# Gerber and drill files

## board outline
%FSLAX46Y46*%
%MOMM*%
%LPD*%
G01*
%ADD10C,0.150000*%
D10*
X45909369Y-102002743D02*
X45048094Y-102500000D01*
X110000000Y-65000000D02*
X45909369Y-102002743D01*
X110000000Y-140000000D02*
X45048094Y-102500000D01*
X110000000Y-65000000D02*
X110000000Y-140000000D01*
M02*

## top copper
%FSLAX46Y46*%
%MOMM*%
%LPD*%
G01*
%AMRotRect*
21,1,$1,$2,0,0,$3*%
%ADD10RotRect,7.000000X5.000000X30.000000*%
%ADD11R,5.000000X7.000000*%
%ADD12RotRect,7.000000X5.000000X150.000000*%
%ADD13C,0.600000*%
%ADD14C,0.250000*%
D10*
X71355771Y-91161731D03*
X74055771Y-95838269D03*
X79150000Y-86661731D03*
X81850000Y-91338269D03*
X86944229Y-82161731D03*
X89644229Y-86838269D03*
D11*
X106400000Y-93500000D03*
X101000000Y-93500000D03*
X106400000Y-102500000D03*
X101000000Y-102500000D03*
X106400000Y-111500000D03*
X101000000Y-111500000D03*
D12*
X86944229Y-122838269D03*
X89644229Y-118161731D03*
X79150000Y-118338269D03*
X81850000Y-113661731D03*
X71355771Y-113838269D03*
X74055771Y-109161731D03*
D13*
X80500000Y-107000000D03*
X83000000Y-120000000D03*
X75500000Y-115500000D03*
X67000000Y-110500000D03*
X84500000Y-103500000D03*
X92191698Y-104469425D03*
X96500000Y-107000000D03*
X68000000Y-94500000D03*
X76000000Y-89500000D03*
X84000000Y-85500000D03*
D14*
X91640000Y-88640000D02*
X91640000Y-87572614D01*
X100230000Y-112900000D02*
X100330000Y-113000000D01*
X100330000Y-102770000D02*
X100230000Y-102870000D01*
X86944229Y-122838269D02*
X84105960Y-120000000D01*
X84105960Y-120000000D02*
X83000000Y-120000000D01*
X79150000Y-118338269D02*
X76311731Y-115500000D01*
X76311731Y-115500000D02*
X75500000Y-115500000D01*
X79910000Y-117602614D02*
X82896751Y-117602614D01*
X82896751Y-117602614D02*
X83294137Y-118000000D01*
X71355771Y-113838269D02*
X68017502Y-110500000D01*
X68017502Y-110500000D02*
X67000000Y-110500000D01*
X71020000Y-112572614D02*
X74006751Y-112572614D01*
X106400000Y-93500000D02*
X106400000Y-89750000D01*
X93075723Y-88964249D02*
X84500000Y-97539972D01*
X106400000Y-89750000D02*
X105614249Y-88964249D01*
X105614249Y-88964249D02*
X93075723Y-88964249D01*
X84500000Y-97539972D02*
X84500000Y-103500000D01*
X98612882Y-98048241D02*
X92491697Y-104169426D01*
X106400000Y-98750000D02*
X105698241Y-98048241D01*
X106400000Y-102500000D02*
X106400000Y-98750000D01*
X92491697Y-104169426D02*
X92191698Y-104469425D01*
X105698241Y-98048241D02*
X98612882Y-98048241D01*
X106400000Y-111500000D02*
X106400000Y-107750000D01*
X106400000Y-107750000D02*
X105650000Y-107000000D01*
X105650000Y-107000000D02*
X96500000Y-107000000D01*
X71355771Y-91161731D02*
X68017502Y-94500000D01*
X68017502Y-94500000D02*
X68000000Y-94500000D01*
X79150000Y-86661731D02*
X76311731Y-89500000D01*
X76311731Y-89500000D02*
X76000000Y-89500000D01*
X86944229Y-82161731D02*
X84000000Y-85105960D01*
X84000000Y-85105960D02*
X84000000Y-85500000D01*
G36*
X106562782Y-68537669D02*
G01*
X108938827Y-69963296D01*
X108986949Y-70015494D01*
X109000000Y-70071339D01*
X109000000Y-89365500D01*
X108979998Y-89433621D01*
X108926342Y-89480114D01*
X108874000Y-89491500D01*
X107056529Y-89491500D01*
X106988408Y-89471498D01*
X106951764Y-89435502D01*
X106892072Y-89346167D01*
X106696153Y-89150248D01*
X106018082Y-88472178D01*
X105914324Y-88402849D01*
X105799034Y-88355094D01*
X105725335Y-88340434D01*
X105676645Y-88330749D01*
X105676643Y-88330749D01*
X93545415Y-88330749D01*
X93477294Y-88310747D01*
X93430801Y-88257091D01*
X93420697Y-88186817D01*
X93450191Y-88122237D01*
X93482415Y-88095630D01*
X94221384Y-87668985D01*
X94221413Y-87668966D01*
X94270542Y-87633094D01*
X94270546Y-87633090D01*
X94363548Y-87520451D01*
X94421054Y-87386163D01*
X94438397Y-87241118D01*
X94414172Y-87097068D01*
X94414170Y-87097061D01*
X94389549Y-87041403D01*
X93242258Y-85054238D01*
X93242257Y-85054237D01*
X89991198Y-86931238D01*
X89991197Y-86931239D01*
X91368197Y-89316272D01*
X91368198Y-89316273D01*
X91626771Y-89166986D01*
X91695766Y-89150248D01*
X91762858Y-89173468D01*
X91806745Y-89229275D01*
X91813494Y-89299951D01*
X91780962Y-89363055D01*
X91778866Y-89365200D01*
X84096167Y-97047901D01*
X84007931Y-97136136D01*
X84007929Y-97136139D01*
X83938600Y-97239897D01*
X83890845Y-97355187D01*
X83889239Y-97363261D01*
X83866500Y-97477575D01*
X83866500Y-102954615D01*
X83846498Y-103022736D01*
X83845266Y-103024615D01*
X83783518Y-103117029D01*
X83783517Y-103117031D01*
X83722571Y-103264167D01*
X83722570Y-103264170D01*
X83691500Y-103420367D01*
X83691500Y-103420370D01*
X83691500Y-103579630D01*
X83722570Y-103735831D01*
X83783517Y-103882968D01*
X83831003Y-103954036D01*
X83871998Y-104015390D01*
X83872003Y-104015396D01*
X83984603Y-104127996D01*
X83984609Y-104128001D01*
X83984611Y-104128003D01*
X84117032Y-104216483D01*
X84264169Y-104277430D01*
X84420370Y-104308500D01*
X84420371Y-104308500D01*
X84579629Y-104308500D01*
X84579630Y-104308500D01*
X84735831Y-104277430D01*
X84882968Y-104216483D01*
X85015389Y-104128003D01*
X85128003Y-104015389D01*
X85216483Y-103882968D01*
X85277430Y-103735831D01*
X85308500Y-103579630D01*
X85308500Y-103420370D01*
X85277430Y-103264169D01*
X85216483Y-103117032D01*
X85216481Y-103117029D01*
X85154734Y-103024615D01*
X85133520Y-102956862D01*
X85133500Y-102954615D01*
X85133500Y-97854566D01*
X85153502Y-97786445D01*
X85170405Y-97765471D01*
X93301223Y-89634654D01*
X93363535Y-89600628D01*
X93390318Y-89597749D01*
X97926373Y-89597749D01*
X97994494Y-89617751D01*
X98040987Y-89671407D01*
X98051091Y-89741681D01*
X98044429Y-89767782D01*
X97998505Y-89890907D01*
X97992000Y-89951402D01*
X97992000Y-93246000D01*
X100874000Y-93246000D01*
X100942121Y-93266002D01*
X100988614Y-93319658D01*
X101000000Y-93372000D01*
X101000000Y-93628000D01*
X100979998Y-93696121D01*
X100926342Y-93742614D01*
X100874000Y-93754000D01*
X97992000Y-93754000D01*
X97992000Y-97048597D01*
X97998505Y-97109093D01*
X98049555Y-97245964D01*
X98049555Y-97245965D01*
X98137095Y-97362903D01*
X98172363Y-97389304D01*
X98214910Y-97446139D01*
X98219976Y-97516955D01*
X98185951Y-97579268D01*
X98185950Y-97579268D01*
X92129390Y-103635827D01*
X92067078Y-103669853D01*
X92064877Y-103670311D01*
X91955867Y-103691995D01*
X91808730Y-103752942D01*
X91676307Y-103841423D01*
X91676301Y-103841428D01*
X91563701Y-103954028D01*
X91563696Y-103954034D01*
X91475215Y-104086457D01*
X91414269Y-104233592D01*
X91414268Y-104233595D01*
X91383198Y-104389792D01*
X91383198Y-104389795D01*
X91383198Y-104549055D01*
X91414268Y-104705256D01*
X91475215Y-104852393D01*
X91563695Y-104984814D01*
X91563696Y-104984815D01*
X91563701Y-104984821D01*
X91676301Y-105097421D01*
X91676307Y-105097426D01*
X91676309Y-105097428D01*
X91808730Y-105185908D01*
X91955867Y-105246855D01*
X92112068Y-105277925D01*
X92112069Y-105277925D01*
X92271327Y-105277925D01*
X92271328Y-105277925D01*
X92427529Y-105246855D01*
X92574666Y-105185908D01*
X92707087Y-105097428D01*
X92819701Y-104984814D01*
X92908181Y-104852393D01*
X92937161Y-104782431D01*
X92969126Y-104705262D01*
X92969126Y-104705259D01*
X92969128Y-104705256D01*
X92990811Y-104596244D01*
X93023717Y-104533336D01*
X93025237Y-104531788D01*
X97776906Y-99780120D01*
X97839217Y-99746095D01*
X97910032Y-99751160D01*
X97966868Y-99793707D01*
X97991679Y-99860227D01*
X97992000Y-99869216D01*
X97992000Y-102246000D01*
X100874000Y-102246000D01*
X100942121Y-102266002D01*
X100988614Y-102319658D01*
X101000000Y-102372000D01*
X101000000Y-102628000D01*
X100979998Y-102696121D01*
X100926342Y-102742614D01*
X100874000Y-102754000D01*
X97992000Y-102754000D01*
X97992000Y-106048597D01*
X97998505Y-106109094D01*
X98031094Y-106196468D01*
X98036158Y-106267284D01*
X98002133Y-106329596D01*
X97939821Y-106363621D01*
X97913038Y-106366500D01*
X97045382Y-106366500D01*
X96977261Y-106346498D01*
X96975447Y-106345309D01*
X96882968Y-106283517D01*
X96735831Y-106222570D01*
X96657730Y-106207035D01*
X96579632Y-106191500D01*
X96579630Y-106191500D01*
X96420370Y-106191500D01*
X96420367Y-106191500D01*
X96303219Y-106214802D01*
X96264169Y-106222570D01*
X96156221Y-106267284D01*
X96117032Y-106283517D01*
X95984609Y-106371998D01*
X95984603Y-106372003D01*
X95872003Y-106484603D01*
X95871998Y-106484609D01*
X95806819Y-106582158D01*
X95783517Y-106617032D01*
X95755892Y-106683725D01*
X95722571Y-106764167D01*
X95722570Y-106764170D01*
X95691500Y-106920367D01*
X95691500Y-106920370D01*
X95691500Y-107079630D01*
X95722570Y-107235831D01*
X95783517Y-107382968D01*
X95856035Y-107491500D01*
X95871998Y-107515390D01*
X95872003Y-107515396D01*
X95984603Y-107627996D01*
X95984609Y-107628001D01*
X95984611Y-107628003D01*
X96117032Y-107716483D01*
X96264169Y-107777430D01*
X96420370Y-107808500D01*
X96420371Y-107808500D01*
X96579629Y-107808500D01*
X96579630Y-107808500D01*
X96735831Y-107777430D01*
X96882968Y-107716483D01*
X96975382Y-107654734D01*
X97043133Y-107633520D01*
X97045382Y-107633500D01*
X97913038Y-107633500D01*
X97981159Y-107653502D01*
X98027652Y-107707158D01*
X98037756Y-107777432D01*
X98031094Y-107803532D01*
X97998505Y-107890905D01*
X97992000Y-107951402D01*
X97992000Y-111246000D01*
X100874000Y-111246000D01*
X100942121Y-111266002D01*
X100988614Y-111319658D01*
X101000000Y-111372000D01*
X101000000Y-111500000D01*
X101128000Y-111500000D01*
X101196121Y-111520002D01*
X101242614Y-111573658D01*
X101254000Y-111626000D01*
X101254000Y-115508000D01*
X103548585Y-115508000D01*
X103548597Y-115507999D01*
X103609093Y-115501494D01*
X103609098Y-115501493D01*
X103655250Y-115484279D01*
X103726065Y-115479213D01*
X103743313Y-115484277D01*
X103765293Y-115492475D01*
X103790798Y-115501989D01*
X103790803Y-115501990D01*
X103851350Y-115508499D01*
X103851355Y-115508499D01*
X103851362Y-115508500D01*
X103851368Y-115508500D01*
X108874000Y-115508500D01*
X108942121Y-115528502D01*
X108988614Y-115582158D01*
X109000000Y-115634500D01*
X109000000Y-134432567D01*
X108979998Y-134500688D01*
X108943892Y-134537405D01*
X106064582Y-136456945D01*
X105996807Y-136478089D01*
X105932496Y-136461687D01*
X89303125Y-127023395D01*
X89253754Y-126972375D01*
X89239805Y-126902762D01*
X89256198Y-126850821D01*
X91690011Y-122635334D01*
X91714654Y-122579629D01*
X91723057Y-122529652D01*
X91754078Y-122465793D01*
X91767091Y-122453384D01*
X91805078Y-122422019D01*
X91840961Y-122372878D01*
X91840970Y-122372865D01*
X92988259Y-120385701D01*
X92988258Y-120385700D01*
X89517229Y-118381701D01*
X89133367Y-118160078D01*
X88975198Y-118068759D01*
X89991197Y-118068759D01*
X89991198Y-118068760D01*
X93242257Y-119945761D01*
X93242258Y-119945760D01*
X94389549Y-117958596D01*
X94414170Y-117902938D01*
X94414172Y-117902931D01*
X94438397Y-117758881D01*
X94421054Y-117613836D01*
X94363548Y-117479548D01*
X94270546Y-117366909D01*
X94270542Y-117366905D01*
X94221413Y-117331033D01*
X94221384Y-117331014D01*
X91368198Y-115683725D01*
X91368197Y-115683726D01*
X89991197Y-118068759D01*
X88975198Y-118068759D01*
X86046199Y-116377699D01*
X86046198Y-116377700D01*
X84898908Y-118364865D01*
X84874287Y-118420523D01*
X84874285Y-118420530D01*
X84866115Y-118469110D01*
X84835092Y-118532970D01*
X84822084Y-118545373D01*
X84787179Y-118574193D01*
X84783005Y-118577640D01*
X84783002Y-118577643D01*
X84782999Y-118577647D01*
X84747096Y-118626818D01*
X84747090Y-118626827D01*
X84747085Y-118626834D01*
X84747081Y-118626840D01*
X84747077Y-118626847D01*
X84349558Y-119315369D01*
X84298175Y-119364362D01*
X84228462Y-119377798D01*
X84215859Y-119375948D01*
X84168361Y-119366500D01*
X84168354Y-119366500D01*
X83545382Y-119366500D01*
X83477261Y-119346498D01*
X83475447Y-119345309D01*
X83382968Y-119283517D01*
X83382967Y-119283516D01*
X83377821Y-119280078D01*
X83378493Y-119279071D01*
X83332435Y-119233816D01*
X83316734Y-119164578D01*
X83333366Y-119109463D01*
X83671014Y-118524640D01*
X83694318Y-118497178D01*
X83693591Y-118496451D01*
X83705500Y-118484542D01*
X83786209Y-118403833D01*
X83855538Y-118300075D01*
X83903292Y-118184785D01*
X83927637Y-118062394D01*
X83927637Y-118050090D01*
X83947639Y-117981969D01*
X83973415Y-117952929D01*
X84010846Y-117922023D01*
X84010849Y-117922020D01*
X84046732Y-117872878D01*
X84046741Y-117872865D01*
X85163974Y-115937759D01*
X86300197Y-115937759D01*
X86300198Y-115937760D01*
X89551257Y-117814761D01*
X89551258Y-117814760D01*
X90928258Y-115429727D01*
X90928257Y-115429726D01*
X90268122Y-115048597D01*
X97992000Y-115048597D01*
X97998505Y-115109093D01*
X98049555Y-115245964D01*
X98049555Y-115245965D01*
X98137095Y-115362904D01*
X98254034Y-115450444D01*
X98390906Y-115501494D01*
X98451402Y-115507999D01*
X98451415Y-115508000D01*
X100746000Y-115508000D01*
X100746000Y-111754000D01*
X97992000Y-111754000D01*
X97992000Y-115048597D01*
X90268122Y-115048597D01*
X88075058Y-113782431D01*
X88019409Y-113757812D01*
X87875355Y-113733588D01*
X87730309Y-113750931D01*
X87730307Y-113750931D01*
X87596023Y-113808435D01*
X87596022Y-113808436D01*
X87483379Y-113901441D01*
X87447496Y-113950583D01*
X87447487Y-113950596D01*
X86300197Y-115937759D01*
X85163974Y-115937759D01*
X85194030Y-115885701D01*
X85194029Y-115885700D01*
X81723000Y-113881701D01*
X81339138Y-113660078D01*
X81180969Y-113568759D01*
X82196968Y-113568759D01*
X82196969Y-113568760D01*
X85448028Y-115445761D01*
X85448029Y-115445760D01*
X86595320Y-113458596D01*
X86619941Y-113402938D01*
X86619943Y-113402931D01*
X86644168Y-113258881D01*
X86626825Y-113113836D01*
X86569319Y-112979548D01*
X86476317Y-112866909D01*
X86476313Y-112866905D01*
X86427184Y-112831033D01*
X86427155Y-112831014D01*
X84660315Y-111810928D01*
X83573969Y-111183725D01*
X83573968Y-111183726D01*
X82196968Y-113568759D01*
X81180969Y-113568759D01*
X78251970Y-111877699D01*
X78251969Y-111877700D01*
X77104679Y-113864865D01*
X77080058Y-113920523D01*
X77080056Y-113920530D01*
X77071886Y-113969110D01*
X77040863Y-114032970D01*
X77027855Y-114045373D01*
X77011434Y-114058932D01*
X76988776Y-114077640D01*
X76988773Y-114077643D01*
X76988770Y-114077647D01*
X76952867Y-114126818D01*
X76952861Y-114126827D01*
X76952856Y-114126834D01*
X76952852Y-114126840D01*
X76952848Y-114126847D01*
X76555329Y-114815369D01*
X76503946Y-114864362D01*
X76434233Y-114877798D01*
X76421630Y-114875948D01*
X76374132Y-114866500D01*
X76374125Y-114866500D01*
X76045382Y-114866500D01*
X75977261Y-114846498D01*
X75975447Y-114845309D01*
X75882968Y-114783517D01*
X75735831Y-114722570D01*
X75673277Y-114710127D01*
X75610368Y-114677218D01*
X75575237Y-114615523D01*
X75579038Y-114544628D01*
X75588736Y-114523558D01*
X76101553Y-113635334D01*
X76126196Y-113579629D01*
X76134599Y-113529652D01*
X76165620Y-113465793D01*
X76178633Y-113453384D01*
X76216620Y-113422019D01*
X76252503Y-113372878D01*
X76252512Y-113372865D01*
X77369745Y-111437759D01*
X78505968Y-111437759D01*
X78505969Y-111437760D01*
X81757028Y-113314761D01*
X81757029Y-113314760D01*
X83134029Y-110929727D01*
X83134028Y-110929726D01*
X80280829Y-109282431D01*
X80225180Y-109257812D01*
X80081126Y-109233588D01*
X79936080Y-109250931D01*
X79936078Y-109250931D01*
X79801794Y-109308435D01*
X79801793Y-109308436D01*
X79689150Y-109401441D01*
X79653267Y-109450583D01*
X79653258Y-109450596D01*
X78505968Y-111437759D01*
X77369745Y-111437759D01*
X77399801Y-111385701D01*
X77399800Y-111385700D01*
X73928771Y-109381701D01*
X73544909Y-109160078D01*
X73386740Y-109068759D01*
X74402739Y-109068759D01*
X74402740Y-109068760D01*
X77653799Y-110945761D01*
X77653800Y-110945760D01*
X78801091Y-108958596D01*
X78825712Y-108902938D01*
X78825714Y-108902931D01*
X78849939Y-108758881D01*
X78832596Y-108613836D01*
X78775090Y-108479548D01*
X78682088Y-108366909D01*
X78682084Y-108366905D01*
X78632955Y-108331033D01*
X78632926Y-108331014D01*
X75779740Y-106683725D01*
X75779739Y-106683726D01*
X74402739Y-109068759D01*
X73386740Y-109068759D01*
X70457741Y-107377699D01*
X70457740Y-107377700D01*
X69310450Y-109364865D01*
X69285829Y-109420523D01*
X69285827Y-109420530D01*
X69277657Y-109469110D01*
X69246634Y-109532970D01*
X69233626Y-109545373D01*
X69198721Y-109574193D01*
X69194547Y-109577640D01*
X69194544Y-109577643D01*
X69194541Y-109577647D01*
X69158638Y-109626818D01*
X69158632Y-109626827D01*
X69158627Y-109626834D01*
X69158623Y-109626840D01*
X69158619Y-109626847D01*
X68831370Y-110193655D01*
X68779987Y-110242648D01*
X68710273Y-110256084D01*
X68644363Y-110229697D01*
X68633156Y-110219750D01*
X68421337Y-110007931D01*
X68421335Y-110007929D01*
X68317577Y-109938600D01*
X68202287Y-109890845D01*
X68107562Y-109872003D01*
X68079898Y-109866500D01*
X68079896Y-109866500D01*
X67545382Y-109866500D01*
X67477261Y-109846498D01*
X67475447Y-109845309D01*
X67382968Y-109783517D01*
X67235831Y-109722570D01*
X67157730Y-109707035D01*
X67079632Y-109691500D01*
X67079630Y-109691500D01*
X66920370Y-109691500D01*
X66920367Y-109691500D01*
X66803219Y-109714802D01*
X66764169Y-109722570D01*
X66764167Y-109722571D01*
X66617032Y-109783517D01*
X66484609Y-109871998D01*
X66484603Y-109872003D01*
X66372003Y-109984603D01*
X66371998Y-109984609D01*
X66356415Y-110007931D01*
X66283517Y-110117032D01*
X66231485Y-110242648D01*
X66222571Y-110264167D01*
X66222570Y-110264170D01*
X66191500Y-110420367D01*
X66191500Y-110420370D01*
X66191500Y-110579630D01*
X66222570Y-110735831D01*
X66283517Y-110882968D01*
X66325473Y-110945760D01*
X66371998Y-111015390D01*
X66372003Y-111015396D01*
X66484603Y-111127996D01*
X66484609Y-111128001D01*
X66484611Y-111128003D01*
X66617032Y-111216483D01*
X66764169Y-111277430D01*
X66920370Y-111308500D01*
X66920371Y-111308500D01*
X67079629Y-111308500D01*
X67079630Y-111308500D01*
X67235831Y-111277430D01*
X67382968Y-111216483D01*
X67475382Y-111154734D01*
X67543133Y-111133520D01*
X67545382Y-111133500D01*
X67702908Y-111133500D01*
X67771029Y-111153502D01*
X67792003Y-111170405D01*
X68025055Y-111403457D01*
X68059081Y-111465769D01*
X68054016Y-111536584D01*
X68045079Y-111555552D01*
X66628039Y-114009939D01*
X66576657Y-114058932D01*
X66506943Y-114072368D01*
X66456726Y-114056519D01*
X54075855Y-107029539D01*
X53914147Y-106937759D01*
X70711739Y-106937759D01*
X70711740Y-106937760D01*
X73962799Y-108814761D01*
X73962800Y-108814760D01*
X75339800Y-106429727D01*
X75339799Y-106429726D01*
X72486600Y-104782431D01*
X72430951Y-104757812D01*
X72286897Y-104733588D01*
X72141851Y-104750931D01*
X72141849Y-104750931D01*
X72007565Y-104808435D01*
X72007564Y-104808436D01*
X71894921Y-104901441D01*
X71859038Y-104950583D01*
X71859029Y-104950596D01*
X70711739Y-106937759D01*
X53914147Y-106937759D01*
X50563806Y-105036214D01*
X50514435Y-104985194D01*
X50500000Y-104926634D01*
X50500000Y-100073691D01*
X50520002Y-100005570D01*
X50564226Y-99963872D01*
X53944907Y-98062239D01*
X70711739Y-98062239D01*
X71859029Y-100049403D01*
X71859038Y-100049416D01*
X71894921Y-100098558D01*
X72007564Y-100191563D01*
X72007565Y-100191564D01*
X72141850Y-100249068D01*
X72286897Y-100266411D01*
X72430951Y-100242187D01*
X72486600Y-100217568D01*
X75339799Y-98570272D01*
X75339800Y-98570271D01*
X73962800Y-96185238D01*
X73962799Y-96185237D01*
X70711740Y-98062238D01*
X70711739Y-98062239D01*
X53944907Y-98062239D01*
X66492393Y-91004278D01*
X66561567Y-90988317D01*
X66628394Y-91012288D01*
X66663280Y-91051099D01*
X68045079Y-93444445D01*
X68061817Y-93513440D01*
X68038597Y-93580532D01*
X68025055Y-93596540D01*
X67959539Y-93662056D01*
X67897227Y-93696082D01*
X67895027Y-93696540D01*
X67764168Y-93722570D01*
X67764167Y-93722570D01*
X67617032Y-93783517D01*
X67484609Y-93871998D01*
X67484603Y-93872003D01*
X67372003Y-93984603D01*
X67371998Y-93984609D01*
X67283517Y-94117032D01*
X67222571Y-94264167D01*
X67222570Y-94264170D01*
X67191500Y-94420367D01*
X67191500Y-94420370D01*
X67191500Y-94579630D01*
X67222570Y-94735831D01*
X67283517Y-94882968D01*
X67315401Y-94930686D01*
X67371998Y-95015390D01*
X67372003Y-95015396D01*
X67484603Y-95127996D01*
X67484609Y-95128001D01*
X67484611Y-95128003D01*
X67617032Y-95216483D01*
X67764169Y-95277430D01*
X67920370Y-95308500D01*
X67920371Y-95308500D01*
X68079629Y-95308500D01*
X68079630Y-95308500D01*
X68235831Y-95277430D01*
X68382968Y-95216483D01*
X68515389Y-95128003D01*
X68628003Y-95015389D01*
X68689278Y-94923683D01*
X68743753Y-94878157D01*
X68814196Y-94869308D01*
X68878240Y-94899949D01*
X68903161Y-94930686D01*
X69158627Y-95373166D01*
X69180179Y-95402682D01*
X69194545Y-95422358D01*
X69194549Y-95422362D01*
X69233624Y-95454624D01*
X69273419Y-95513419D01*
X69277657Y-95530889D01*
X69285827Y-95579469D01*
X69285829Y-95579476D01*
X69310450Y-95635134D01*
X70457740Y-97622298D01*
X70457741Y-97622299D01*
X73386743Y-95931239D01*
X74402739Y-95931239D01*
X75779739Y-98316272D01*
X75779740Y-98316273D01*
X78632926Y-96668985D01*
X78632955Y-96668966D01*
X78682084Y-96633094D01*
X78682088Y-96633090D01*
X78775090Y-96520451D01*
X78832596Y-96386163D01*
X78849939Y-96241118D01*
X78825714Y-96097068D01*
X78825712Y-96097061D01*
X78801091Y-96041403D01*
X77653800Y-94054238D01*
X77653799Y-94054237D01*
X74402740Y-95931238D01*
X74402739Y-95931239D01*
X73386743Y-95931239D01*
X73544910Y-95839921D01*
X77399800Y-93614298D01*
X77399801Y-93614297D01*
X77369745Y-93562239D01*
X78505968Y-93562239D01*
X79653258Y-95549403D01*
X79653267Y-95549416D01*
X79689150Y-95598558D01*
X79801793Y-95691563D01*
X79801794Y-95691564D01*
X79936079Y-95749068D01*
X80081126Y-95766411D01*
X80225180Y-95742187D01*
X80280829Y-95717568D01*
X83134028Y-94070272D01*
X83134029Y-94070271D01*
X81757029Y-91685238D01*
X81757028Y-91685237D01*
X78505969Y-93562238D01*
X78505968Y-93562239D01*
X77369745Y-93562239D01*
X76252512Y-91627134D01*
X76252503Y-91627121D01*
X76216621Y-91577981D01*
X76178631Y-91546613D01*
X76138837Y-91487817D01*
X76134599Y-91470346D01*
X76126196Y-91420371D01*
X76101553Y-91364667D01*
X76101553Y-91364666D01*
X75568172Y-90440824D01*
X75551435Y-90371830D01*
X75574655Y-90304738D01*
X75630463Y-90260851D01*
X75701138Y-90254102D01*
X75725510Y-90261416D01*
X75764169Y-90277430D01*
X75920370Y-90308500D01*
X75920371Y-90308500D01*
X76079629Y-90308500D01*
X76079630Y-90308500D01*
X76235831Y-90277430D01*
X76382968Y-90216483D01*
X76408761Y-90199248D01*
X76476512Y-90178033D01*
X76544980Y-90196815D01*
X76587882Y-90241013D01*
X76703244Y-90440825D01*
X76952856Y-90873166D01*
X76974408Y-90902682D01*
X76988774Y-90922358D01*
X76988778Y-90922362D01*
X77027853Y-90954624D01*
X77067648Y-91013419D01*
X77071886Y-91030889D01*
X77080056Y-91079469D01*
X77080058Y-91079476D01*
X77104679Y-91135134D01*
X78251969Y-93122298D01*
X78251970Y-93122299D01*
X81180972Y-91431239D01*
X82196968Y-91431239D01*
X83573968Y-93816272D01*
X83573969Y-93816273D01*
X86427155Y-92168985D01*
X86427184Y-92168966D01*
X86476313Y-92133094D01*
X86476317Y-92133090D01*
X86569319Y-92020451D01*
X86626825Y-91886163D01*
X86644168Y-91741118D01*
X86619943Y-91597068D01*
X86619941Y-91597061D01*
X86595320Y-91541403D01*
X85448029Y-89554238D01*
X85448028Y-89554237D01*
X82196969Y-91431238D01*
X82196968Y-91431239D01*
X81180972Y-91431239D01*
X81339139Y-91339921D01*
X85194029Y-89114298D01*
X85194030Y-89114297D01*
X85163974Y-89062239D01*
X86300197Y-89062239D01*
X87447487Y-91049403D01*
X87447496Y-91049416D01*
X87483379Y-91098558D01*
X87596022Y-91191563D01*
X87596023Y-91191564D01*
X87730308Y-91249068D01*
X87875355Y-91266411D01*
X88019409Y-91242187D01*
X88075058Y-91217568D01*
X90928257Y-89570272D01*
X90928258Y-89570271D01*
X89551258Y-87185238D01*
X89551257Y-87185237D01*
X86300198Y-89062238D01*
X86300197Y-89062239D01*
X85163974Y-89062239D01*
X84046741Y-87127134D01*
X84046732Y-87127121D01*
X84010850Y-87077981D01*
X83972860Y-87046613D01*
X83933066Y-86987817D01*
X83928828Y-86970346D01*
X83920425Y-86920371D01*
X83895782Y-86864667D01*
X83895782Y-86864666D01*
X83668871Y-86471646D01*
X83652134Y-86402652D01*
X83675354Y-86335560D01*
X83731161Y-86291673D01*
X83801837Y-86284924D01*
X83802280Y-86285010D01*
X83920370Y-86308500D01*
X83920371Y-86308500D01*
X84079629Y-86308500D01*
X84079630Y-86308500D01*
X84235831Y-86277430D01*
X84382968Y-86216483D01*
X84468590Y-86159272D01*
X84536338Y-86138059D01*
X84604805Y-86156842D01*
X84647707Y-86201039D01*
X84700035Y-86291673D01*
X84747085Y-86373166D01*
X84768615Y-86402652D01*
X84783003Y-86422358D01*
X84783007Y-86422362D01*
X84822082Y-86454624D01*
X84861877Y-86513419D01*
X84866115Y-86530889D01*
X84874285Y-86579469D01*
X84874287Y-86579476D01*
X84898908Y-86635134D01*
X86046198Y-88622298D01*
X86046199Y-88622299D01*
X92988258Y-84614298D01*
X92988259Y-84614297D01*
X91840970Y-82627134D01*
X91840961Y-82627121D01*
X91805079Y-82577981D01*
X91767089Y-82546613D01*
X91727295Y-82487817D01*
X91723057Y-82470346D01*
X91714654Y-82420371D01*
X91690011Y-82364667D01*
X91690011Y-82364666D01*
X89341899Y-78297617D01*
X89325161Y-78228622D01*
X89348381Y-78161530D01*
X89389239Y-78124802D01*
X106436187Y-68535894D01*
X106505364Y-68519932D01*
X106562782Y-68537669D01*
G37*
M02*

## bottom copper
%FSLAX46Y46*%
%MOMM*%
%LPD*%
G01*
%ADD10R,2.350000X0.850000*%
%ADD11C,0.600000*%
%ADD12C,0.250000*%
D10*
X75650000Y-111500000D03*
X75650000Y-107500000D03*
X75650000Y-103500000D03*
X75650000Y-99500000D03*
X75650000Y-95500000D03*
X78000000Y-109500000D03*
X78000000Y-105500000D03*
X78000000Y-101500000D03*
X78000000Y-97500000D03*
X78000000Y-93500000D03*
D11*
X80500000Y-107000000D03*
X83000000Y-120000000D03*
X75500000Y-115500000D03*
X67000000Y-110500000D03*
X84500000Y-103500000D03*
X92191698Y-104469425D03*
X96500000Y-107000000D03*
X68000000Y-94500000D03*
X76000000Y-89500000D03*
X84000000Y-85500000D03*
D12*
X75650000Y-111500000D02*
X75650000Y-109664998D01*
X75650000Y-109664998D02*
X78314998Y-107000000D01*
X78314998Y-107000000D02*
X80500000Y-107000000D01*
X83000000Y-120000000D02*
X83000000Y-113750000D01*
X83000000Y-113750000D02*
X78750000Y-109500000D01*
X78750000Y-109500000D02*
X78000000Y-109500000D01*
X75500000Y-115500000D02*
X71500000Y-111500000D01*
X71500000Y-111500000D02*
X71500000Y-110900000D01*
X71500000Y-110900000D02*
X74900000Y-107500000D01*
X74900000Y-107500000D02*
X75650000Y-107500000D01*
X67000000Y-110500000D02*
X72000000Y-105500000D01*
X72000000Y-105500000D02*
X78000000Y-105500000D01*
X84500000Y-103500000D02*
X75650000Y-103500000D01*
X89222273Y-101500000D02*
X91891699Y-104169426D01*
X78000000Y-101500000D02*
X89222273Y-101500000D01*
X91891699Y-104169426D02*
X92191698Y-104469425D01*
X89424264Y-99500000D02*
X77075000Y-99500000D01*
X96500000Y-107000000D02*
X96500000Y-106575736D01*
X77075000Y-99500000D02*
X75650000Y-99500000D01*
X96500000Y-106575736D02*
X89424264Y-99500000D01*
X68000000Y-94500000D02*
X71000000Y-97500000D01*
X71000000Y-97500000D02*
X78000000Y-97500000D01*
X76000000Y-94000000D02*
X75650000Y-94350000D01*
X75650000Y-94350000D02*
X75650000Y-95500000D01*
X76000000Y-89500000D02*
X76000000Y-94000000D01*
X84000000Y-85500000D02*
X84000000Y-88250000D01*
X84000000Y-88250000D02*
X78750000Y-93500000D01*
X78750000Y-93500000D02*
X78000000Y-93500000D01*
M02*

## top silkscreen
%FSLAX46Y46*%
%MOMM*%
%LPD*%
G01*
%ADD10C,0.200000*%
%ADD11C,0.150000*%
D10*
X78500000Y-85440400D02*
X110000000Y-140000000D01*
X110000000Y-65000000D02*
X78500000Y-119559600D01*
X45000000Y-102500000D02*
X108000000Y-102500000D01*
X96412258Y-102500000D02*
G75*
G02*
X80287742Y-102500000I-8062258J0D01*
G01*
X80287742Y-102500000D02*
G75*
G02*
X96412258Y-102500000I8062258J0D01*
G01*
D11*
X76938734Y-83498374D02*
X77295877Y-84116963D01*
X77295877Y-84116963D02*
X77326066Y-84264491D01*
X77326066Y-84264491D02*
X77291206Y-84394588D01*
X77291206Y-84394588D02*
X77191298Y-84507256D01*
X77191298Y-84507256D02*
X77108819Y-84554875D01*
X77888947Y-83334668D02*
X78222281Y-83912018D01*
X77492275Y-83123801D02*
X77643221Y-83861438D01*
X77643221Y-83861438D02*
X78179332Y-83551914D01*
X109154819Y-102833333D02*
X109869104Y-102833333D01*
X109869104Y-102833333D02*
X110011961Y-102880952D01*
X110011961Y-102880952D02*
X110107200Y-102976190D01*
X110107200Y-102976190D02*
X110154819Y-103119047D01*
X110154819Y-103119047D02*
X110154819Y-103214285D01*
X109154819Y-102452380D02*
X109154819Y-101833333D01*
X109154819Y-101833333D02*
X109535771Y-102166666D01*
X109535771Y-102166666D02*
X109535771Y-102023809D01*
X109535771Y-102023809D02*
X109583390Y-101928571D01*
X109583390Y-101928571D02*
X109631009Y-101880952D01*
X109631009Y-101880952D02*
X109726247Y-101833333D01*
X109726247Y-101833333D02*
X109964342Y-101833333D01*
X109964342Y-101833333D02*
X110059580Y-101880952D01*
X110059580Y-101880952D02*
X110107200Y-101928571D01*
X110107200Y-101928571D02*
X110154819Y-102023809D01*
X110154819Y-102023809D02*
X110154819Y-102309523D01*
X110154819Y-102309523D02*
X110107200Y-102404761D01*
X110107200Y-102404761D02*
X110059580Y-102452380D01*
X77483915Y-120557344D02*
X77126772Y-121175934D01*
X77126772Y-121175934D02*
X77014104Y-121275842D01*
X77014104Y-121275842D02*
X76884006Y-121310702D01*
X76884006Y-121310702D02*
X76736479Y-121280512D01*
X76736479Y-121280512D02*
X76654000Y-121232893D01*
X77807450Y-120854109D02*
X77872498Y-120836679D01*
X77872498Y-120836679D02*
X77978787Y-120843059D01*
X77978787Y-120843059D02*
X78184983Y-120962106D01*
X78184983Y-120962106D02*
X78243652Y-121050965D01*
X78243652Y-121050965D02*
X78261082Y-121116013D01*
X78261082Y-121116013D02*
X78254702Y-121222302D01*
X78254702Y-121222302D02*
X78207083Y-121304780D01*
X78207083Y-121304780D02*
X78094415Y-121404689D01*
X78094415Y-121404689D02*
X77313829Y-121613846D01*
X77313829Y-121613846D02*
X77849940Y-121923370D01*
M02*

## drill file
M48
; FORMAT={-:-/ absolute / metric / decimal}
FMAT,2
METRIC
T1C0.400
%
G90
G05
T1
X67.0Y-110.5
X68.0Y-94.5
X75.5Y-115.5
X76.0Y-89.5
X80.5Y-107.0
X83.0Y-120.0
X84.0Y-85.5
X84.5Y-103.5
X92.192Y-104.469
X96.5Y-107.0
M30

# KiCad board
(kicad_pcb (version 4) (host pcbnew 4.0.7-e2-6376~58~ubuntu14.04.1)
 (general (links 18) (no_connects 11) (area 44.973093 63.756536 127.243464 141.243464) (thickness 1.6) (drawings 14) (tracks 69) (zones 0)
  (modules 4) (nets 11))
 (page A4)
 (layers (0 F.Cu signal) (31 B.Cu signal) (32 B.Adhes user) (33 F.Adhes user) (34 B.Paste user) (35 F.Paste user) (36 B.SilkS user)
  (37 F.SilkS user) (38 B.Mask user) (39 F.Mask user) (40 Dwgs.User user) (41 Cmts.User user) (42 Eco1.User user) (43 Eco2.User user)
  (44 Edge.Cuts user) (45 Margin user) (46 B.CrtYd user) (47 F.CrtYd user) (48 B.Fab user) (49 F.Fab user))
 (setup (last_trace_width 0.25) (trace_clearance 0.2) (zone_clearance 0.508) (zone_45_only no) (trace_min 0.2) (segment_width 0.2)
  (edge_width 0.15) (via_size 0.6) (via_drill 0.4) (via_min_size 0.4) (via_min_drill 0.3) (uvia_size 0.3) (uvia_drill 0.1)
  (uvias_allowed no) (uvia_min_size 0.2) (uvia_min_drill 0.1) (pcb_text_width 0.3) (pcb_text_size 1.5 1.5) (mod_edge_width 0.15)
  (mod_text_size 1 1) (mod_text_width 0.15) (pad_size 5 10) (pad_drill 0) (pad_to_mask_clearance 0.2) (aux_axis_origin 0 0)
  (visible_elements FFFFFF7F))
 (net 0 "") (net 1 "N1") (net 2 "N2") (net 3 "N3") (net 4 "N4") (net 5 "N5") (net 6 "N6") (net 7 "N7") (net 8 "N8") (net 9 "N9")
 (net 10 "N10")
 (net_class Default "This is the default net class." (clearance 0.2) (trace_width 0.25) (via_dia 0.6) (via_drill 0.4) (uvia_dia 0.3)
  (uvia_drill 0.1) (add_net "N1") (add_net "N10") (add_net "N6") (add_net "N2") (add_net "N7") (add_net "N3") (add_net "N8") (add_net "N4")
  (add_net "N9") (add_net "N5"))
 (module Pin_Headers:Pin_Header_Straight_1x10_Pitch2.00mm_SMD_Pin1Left (layer B.Cu) (at 76.825 102.5)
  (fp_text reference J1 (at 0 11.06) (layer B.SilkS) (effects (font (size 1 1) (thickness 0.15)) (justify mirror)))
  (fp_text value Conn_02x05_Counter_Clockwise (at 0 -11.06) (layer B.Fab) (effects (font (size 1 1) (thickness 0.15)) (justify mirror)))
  (pad 1 smd rect (at -1.175 9) (size 2.35 0.85) (layers B.Cu B.Paste B.Mask) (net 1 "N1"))
  (pad 3 smd rect (at -1.175 5) (size 2.35 0.85) (layers B.Cu B.Paste B.Mask) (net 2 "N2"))
  (pad 5 smd rect (at -1.175 1) (size 2.35 0.85) (layers B.Cu B.Paste B.Mask) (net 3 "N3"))
  (pad 7 smd rect (at -1.175 -3) (size 2.35 0.85) (layers B.Cu B.Paste B.Mask) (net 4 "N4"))
  (pad 9 smd rect (at -1.175 -7) (size 2.35 0.85) (layers B.Cu B.Paste B.Mask) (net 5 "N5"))
  (pad 2 smd rect (at 1.175 7) (size 2.35 0.85) (layers B.Cu B.Paste B.Mask) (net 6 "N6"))
  (pad 4 smd rect (at 1.175 3) (size 2.35 0.85) (layers B.Cu B.Paste B.Mask) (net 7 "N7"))
  (pad 6 smd rect (at 1.175 -1) (size 2.35 0.85) (layers B.Cu B.Paste B.Mask) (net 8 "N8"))
  (pad 8 smd rect (at 1.175 -5) (size 2.35 0.85) (layers B.Cu B.Paste B.Mask) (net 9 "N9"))
  (pad 10 smd rect (at 1.175 -9) (size 2.35 0.85) (layers B.Cu B.Paste B.Mask) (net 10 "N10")))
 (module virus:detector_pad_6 (layer F.Cu) (at 80.5 89 30)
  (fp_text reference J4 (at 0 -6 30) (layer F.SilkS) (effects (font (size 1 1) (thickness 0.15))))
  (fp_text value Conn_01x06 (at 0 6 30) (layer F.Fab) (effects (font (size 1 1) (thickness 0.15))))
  (pad 1 smd rect (at -9 -2.7 30) (size 7 5) (layers F.Cu F.Paste F.Mask) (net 9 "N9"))
  (pad 2 smd rect (at -9 2.7 30) (size 7 5) (layers F.Cu F.Paste F.Mask) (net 1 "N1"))
  (pad 3 smd rect (at 0 -2.7 30) (size 7 5) (layers F.Cu F.Paste F.Mask) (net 5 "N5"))
  (pad 4 smd rect (at 0 2.7 30) (size 7 5) (layers F.Cu F.Paste F.Mask) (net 1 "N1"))
  (pad 5 smd rect (at 9 -2.7 30) (size 7 5) (layers F.Cu F.Paste F.Mask) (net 10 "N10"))
  (pad 6 smd rect (at 9 2.7 30) (size 7 5) (layers F.Cu F.Paste F.Mask) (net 1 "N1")))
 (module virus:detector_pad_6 (layer F.Cu) (at 103.7 102.5 270)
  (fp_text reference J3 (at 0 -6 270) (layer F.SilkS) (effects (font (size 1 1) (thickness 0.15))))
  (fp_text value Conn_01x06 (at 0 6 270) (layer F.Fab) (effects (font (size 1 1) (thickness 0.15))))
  (pad 1 smd rect (at -9 -2.7 270) (size 7 5) (layers F.Cu F.Paste F.Mask) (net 3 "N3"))
  (pad 2 smd rect (at -9 2.7 270) (size 7 5) (layers F.Cu F.Paste F.Mask) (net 1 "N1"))
  (pad 3 smd rect (at 0 -2.7 270) (size 7 5) (layers F.Cu F.Paste F.Mask) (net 8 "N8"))
  (pad 4 smd rect (at 0 2.7 270) (size 7 5) (layers F.Cu F.Paste F.Mask) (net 1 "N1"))
  (pad 5 smd rect (at 9 -2.7 270) (size 7 5) (layers F.Cu F.Paste F.Mask) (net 4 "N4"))
  (pad 6 smd rect (at 9 2.7 270) (size 7 5) (layers F.Cu F.Paste F.Mask) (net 1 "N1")))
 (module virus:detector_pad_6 (layer F.Cu) (at 80.5 116 150)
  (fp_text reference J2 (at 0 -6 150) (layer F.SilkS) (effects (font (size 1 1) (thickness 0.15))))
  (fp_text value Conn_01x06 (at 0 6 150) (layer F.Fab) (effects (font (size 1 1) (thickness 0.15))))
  (pad 1 smd rect (at -9 -2.7 150) (size 7 5) (layers F.Cu F.Paste F.Mask) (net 6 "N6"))
  (pad 2 smd rect (at -9 2.7 150) (size 7 5) (layers F.Cu F.Paste F.Mask) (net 1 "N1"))
  (pad 3 smd rect (at 0 -2.7 150) (size 7 5) (layers F.Cu F.Paste F.Mask) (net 2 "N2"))
  (pad 4 smd rect (at 0 2.7 150) (size 7 5) (layers F.Cu F.Paste F.Mask) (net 1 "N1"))
  (pad 5 smd rect (at 9 -2.7 150) (size 7 5) (layers F.Cu F.Paste F.Mask) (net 7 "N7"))
  (pad 6 smd rect (at 9 2.7 150) (size 7 5) (layers F.Cu F.Paste F.Mask) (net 1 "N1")))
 (gr_line (start 45.909369 102.002743) (end 45.048094 102.5) (layer Edge.Cuts) (width 0.15))
 (gr_line (start 78.5 85.4404) (end 110 140) (layer F.SilkS) (width 0.2))
 (gr_line (start 110 65) (end 78.5 119.5596) (layer F.SilkS) (width 0.2))
 (gr_line (start 45 102.5) (end 108 102.5) (layer F.SilkS) (width 0.2))
 (gr_circle (center 88.35 102.5) (end 95.35 106.5) (layer F.SilkS) (width 0.2))
 (gr_line (start 110 65) (end 45.909369 102.002743) (layer Edge.Cuts) (width 0.15))
 (gr_line (start 110 140) (end 45.048094 102.5) (layer Edge.Cuts) (width 0.15))
 (gr_line (start 110 65) (end 110 140) (layer Edge.Cuts) (width 0.15))
 (segment (start 75.65 111.5) (end 75.65 109.664998) (width 0.25) (layer B.Cu) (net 1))
 (segment (start 75.65 109.664998) (end 78.314998 107) (width 0.25) (layer B.Cu) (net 1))
 (segment (start 78.314998 107) (end 80.5 107) (width 0.25) (layer B.Cu) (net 1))
 (via (at 80.5 107) (size 0.6) (drill 0.4) (layers F.Cu B.Cu) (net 1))
 (segment (start 91.64 88.64) (end 91.64 87.572614) (width 0.25) (layer F.Cu) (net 1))
 (segment (start 100.23 112.9) (end 100.33 113) (width 0.25) (layer F.Cu) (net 1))
 (segment (start 100.33 102.77) (end 100.23 102.87) (width 0.25) (layer F.Cu) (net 1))
 (segment (start 83 120) (end 83 113.75) (width 0.25) (layer B.Cu) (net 6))
 (segment (start 83 113.75) (end 78.75 109.5) (width 0.25) (layer B.Cu) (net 6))
 (segment (start 78.75 109.5) (end 78 109.5) (width 0.25) (layer B.Cu) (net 6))
 (segment (start 86.944229 122.838269) (end 84.10596 120) (width 0.25) (layer F.Cu) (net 6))
 (segment (start 84.10596 120) (end 83 120) (width 0.25) (layer F.Cu) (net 6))
 (via (at 83 120) (size 0.6) (drill 0.4) (layers F.Cu B.Cu) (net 6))
 (segment (start 75.5 115.5) (end 71.5 111.5) (width 0.25) (layer B.Cu) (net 2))
 (segment (start 71.5 111.5) (end 71.5 110.9) (width 0.25) (layer B.Cu) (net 2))
 (segment (start 71.5 110.9) (end 74.9 107.5) (width 0.25) (layer B.Cu) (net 2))
 (segment (start 74.9 107.5) (end 75.65 107.5) (width 0.25) (layer B.Cu) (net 2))
 (segment (start 79.15 118.338269) (end 76.311731 115.5) (width 0.25) (layer F.Cu) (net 2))
 (segment (start 76.311731 115.5) (end 75.5 115.5) (width 0.25) (layer F.Cu) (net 2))
 (via (at 75.5 115.5) (size 0.6) (drill 0.4) (layers F.Cu B.Cu) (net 2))
 (segment (start 79.91 117.602614) (end 82.896751 117.602614) (width 0.25) (layer F.Cu) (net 2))
 (segment (start 82.896751 117.602614) (end 83.294137 118) (width 0.25) (layer F.Cu) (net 2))
 (segment (start 67 110.5) (end 72 105.5) (width 0.25) (layer B.Cu) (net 7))
 (segment (start 72 105.5) (end 78 105.5) (width 0.25) (layer B.Cu) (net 7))
 (segment (start 71.355771 113.838269) (end 68.017502 110.5) (width 0.25) (layer F.Cu) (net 7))
 (segment (start 68.017502 110.5) (end 67 110.5) (width 0.25) (layer F.Cu) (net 7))
 (via (at 67 110.5) (size 0.6) (drill 0.4) (layers F.Cu B.Cu) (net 7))
 (segment (start 71.02 112.572614) (end 74.006751 112.572614) (width 0.25) (layer F.Cu) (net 7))
 (segment (start 106.4 93.5) (end 106.4 89.75) (width 0.25) (layer F.Cu) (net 3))
 (segment (start 93.075723 88.964249) (end 84.5 97.539972) (width 0.25) (layer F.Cu) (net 3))
 (segment (start 106.4 89.75) (end 105.614249 88.964249) (width 0.25) (layer F.Cu) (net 3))
 (segment (start 105.614249 88.964249) (end 93.075723 88.964249) (width 0.25) (layer F.Cu) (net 3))
 (segment (start 84.5 97.539972) (end 84.5 103.5) (width 0.25) (layer F.Cu) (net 3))
 (segment (start 84.5 103.5) (end 75.65 103.5) (width 0.25) (layer B.Cu) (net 3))
 (via (at 84.5 103.5) (size 0.6) (drill 0.4) (layers F.Cu B.Cu) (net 3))
 (segment (start 89.222273 101.5) (end 91.891699 104.169426) (width 0.25) (layer B.Cu) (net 8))
 (segment (start 98.612882 98.048241) (end 92.491697 104.169426) (width 0.25) (layer F.Cu) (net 8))
 (segment (start 106.4 98.75) (end 105.698241 98.048241) (width 0.25) (layer F.Cu) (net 8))
 (segment (start 106.4 102.5) (end 106.4 98.75) (width 0.25) (layer F.Cu) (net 8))
 (segment (start 78 101.5) (end 89.222273 101.5) (width 0.25) (layer B.Cu) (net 8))
 (segment (start 92.491697 104.169426) (end 92.191698 104.469425) (width 0.25) (layer F.Cu) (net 8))
 (via (at 92.191698 104.469425) (size 0.6) (drill 0.4) (layers F.Cu B.Cu) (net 8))
 (segment (start 91.891699 104.169426) (end 92.191698 104.469425) (width 0.25) (layer B.Cu) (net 8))
 (segment (start 105.698241 98.048241) (end 98.612882 98.048241) (width 0.25) (layer F.Cu) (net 8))
 (segment (start 89.424264 99.5) (end 77.075 99.5) (width 0.25) (layer B.Cu) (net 4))
 (segment (start 96.5 107) (end 96.5 106.575736) (width 0.25) (layer B.Cu) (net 4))
 (segment (start 77.075 99.5) (end 75.65 99.5) (width 0.25) (layer B.Cu) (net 4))
 (segment (start 96.5 106.575736) (end 89.424264 99.5) (width 0.25) (layer B.Cu) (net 4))
 (segment (start 106.4 111.5) (end 106.4 107.75) (width 0.25) (layer F.Cu) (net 4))
 (segment (start 106.4 107.75) (end 105.65 107) (width 0.25) (layer F.Cu) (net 4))
 (segment (start 105.65 107) (end 96.5 107) (width 0.25) (layer F.Cu) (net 4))
 (via (at 96.5 107) (size 0.6) (drill 0.4) (layers F.Cu B.Cu) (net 4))
 (segment (start 68 94.5) (end 71 97.5) (width 0.25) (layer B.Cu) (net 9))
 (segment (start 71 97.5) (end 78 97.5) (width 0.25) (layer B.Cu) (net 9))
 (segment (start 71.355771 91.161731) (end 68.017502 94.5) (width 0.25) (layer F.Cu) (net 9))
 (segment (start 68.017502 94.5) (end 68 94.5) (width 0.25) (layer F.Cu) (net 9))
 (via (at 68 94.5) (size 0.6) (drill 0.4) (layers F.Cu B.Cu) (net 9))
 (segment (start 76 94) (end 75.65 94.35) (width 0.25) (layer B.Cu) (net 5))
 (segment (start 75.65 94.35) (end 75.65 95.5) (width 0.25) (layer B.Cu) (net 5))
 (segment (start 76 89.5) (end 76 94) (width 0.25) (layer B.Cu) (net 5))
 (segment (start 79.15 86.661731) (end 76.311731 89.5) (width 0.25) (layer F.Cu) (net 5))
 (segment (start 76.311731 89.5) (end 76 89.5) (width 0.25) (layer F.Cu) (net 5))
 (via (at 76 89.5) (size 0.6) (drill 0.4) (layers F.Cu B.Cu) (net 5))
 (segment (start 84 85.5) (end 84 88.25) (width 0.25) (layer B.Cu) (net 10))
 (segment (start 84 88.25) (end 78.75 93.5) (width 0.25) (layer B.Cu) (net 10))
 (segment (start 78.75 93.5) (end 78 93.5) (width 0.25) (layer B.Cu) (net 10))
 (segment (start 86.944229 82.161731) (end 84 85.10596) (width 0.25) (layer F.Cu) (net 10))
 (segment (start 84 85.10596) (end 84 85.5) (width 0.25) (layer F.Cu) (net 10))
 (via (at 84 85.5) (size 0.6) (drill 0.4) (layers F.Cu B.Cu) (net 10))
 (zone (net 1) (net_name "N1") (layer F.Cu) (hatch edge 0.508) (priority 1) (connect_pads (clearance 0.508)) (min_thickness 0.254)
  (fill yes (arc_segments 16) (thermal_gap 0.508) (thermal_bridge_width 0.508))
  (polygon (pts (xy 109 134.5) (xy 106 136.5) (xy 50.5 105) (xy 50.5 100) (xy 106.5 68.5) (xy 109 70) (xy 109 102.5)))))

